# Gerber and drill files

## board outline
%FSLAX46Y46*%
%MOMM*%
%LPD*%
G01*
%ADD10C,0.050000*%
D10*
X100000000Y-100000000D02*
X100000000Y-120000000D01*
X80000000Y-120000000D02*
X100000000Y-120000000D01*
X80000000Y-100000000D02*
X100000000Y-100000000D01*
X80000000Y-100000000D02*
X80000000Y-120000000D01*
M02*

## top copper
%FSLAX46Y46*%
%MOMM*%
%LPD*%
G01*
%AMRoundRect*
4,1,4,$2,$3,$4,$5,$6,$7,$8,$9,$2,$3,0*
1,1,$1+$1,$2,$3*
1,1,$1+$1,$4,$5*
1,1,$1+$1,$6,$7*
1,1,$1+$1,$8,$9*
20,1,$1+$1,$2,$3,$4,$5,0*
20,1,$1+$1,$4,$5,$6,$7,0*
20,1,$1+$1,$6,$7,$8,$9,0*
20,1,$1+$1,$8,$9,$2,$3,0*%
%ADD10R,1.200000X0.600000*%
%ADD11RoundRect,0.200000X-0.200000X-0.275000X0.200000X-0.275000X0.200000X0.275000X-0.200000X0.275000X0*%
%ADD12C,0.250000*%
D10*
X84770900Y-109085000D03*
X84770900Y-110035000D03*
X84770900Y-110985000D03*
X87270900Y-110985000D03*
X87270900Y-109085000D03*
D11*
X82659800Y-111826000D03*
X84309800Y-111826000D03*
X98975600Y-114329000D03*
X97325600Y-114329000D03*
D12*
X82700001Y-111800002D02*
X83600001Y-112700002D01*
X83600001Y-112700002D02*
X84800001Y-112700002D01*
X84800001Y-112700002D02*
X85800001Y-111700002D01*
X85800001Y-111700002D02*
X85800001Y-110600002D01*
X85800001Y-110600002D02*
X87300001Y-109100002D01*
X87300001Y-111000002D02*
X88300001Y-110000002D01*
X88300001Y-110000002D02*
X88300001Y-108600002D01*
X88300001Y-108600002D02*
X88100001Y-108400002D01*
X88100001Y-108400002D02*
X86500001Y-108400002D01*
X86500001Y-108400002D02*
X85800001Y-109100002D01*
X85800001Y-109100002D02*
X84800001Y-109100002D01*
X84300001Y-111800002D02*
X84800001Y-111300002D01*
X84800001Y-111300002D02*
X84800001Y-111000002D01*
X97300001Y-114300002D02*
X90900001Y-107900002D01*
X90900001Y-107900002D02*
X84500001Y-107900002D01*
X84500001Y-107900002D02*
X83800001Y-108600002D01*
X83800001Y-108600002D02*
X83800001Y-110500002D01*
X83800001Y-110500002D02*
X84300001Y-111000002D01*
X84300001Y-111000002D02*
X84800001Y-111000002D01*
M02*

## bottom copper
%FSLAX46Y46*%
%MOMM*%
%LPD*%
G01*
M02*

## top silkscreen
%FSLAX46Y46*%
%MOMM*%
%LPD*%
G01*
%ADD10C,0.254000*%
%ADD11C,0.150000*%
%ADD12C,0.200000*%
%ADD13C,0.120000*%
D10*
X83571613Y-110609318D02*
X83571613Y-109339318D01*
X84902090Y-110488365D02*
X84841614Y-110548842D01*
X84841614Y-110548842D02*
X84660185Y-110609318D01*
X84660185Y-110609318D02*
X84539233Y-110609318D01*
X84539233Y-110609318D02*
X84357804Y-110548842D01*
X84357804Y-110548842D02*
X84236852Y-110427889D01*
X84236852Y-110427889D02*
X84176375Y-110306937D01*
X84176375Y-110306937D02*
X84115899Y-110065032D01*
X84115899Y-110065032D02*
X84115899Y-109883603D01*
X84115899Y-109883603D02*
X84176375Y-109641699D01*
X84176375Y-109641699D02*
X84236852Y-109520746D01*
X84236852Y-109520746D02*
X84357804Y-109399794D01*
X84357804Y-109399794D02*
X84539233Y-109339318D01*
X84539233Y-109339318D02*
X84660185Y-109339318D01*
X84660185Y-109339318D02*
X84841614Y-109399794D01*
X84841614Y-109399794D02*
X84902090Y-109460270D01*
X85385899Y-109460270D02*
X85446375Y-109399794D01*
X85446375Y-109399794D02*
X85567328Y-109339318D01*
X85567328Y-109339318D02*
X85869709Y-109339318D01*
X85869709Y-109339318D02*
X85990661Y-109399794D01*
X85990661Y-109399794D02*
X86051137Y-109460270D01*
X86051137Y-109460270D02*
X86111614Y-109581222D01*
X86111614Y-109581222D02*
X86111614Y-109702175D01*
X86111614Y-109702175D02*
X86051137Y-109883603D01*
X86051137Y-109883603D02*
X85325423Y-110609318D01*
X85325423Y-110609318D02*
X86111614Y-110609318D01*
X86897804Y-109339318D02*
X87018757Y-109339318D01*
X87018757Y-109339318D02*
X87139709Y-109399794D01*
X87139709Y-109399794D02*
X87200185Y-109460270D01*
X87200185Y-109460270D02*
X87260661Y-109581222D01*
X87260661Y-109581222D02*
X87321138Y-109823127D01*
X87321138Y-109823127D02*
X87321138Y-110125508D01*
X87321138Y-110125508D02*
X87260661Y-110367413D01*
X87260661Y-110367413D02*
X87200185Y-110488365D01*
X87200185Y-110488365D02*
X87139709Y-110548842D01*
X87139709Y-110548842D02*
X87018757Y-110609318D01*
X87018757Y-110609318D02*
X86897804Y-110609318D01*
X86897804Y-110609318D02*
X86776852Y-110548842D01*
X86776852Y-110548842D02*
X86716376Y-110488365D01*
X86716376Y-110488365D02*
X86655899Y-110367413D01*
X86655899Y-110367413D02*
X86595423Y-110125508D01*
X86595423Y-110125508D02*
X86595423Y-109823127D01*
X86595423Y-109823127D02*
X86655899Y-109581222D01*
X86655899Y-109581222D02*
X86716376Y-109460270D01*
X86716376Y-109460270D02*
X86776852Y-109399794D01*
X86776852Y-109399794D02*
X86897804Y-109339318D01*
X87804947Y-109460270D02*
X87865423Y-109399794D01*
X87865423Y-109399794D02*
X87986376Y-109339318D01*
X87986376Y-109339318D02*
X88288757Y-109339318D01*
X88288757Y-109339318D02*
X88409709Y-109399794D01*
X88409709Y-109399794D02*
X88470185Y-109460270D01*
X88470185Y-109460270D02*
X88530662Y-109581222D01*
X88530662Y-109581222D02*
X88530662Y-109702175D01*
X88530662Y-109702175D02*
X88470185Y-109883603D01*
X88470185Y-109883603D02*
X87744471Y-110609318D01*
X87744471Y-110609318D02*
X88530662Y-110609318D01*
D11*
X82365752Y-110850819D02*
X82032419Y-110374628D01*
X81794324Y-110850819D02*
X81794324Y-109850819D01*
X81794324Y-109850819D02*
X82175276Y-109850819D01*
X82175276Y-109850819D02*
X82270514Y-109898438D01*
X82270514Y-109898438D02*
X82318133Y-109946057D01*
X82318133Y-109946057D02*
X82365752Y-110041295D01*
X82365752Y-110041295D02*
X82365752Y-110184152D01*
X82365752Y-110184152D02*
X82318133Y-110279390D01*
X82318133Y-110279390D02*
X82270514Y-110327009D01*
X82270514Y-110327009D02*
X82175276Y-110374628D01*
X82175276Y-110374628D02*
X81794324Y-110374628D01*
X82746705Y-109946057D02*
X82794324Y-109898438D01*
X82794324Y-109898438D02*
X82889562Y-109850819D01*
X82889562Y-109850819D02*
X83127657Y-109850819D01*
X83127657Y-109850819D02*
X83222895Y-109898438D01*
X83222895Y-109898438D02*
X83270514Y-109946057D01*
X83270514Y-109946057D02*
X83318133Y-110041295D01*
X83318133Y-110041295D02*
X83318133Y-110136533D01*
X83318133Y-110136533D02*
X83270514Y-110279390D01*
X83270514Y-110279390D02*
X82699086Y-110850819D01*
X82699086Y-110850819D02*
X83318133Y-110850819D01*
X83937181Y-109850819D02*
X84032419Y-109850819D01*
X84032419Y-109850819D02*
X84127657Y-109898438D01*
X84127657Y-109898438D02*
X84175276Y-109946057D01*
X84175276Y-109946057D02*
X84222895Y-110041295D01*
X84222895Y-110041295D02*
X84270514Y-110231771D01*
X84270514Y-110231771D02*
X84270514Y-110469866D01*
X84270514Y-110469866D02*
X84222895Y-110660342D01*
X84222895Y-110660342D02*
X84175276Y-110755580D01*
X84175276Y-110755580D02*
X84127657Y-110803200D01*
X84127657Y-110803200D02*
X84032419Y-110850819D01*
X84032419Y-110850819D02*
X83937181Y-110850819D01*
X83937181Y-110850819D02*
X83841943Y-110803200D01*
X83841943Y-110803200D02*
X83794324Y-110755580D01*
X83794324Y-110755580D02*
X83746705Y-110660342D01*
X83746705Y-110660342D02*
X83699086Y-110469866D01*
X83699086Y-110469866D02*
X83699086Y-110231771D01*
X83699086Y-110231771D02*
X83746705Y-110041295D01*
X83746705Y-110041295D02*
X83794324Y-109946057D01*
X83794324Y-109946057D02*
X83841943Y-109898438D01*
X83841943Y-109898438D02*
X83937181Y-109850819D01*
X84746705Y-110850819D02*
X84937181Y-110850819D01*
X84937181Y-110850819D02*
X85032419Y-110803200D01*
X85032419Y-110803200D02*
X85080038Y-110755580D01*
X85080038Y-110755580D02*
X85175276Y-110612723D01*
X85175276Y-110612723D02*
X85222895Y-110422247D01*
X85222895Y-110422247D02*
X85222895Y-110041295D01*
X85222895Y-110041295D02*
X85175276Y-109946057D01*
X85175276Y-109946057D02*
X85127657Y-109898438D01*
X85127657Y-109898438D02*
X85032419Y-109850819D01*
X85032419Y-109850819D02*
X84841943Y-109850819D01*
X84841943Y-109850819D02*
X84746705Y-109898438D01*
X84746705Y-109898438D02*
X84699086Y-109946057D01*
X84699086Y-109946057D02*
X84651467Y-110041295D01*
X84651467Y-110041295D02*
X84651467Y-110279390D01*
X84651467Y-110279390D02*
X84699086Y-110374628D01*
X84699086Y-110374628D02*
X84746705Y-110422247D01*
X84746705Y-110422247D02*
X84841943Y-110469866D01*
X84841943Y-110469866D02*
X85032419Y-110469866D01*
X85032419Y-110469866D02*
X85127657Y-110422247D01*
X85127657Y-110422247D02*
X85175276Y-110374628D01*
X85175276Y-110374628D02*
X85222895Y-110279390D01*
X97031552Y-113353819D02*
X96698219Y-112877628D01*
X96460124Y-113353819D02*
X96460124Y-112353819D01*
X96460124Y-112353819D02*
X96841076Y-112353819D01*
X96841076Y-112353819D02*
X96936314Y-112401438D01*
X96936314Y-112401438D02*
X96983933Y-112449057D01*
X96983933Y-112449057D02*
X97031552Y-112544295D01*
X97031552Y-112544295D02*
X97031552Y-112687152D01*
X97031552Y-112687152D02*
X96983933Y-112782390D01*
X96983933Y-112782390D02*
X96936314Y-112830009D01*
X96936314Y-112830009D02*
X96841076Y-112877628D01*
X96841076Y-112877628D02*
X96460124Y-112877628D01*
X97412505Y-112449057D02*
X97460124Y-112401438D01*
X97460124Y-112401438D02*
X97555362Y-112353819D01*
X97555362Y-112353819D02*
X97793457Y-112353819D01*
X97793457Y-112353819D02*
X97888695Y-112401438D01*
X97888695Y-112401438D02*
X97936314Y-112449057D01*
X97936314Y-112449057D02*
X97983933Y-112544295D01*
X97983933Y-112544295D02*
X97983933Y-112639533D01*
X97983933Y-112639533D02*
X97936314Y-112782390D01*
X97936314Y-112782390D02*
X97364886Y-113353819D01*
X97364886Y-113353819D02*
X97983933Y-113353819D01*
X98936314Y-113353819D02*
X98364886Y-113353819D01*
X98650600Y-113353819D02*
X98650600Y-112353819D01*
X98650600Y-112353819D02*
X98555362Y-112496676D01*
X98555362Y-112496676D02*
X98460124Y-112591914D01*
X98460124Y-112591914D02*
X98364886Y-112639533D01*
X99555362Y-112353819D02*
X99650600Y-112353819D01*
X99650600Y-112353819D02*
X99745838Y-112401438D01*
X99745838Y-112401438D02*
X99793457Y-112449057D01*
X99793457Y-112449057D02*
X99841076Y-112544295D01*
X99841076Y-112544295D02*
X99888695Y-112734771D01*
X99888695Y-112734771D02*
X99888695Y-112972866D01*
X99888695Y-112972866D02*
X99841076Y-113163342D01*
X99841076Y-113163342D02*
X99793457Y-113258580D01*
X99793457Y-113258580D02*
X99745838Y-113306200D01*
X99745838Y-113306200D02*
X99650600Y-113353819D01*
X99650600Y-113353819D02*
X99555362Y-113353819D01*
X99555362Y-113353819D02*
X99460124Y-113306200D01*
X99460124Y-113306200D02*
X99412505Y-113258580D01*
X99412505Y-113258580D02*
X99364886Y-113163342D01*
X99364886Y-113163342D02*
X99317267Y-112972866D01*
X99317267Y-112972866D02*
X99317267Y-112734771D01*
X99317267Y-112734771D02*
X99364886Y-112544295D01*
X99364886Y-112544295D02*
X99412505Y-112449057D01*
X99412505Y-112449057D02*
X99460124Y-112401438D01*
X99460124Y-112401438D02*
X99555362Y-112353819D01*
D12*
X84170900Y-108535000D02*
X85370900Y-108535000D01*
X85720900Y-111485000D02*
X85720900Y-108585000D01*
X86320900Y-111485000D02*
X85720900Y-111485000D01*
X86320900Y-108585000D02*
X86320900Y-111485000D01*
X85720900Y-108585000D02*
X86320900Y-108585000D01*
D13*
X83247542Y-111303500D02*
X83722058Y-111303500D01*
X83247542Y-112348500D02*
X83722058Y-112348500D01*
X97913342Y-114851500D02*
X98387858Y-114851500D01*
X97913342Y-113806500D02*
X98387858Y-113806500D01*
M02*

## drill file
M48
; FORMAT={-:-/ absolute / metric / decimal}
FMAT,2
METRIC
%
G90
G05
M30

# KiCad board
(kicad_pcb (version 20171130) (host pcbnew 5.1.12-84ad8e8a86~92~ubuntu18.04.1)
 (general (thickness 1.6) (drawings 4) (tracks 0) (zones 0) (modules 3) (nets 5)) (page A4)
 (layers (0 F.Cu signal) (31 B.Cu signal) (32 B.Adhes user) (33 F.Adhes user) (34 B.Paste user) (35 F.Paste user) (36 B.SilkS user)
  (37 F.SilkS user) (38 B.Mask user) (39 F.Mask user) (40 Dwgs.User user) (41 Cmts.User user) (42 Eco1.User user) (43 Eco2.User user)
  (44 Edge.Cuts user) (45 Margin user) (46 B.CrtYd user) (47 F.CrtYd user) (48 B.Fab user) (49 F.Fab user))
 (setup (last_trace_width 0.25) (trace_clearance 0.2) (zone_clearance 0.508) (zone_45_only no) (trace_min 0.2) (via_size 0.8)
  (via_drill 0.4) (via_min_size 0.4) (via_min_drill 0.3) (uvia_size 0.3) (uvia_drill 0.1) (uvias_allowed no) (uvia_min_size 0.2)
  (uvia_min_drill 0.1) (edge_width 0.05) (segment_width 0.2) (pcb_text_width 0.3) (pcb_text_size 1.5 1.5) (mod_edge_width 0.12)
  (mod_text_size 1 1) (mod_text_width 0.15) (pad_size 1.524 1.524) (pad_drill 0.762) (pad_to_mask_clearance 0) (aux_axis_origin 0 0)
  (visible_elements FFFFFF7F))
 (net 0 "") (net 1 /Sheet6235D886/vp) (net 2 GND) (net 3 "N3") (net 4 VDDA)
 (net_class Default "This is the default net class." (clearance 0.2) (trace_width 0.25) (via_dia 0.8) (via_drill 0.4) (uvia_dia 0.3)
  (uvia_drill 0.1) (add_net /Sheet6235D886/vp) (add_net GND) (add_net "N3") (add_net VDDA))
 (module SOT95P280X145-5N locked (layer F.Cu) (at 86.020900 110.035000)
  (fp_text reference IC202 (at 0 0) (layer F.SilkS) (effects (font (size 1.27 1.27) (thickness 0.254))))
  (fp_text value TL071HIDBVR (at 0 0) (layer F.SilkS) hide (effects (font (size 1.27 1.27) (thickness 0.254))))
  (fp_line (start -1.85 -1.5) (end -0.65 -1.5) (layer F.SilkS) (width 0.2))
  (fp_line (start -0.3 1.45) (end -0.3 -1.45) (layer F.SilkS) (width 0.2))
  (fp_line (start 0.3 1.45) (end -0.3 1.45) (layer F.SilkS) (width 0.2))
  (fp_line (start 0.3 -1.45) (end 0.3 1.45) (layer F.SilkS) (width 0.2))
  (fp_line (start -0.3 -1.45) (end 0.3 -1.45) (layer F.SilkS) (width 0.2))
  (pad 1 smd rect (at -1.25 -0.95 90.000000) (size 0.6 1.2) (layers F.Cu F.Mask F.Paste) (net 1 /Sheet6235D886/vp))
  (pad 2 smd rect (at -1.25 0 90.000000) (size 0.6 1.2) (layers F.Cu F.Mask F.Paste) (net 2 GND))
  (pad 3 smd rect (at -1.25 0.95 90.000000) (size 0.6 1.2) (layers F.Cu F.Mask F.Paste) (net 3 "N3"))
  (pad 4 smd rect (at 1.25 0.95 90.000000) (size 0.6 1.2) (layers F.Cu F.Mask F.Paste) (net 1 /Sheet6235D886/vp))
  (pad 5 smd rect (at 1.25 -0.95 90.000000) (size 0.6 1.2) (layers F.Cu F.Mask F.Paste) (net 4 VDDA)))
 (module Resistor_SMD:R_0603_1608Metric (layer F.Cu) (at 83.484800 111.826000)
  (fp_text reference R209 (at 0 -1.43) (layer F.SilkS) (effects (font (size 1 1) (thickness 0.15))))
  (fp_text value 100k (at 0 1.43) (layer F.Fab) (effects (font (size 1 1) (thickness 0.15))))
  (fp_line (start -0.237258 -0.5225) (end 0.237258 -0.5225) (layer F.SilkS) (width 0.12))
  (fp_line (start -0.237258 0.5225) (end 0.237258 0.5225) (layer F.SilkS) (width 0.12))
  (pad 1 smd roundrect (at -0.825 0) (size 0.8 0.95) (layers F.Cu F.Mask F.Paste) (roundrect_rratio 0.25) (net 4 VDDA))
  (pad 2 smd roundrect (at 0.825 0) (size 0.8 0.95) (layers F.Cu F.Mask F.Paste) (roundrect_rratio 0.25) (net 3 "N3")))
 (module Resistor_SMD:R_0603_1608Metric (layer F.Cu) (at 98.150600 114.329000)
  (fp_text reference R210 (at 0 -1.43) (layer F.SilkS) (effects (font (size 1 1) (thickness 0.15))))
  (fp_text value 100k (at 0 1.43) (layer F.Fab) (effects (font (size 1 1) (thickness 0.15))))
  (fp_line (start -0.237258 0.5225) (end 0.237258 0.5225) (layer F.SilkS) (width 0.12))
  (fp_line (start -0.237258 -0.5225) (end 0.237258 -0.5225) (layer F.SilkS) (width 0.12))
  (pad 2 smd roundrect (at 0.825 0) (size 0.8 0.95) (layers F.Cu F.Mask F.Paste) (roundrect_rratio 0.25) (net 2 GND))
  (pad 1 smd roundrect (at -0.825 0) (size 0.8 0.95) (layers F.Cu F.Mask F.Paste) (roundrect_rratio 0.25) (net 3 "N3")))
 (gr_line (start 100 100) (end 100 120) (layer Edge.Cuts) (width 0.05))
 (gr_line (start 80 120) (end 100 120) (layer Edge.Cuts) (width 0.05))
 (gr_line (start 80 100) (end 100 100) (layer Edge.Cuts) (width 0.05))
 (gr_line (start 80 100) (end 80 120) (layer Edge.Cuts) (width 0.05))
 (segment (start 82.700001 111.800002) (end 83.600001 112.700002) (width 0.250000) (layer F.Cu) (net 4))
 (segment (start 83.600001 112.700002) (end 84.800001 112.700002) (width 0.250000) (layer F.Cu) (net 4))
 (segment (start 84.800001 112.700002) (end 85.800001 111.700002) (width 0.250000) (layer F.Cu) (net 4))
 (segment (start 85.800001 111.700002) (end 85.800001 110.600002) (width 0.250000) (layer F.Cu) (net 4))
 (segment (start 85.800001 110.600002) (end 87.300001 109.100002) (width 0.250000) (layer F.Cu) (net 4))
 (segment (start 87.300001 111.000002) (end 88.300001 110.000002) (width 0.250000) (layer F.Cu) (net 1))
 (segment (start 88.300001 110.000002) (end 88.300001 108.600002) (width 0.250000) (layer F.Cu) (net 1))
 (segment (start 88.300001 108.600002) (end 88.100001 108.400002) (width 0.250000) (layer F.Cu) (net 1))
 (segment (start 88.100001 108.400002) (end 86.500001 108.400002) (width 0.250000) (layer F.Cu) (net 1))
 (segment (start 86.500001 108.400002) (end 85.800001 109.100002) (width 0.250000) (layer F.Cu) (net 1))
 (segment (start 85.800001 109.100002) (end 84.800001 109.100002) (width 0.250000) (layer F.Cu) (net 1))
 (segment (start 84.300001 111.800002) (end 84.800001 111.300002) (width 0.250000) (layer F.Cu) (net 3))
 (segment (start 84.800001 111.300002) (end 84.800001 111.000002) (width 0.250000) (layer F.Cu) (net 3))
 (segment (start 97.300001 114.300002) (end 90.900001 107.900002) (width 0.250000) (layer F.Cu) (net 3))
 (segment (start 90.900001 107.900002) (end 84.500001 107.900002) (width 0.250000) (layer F.Cu) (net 3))
 (segment (start 84.500001 107.900002) (end 83.800001 108.600002) (width 0.250000) (layer F.Cu) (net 3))
 (segment (start 83.800001 108.600002) (end 83.800001 110.500002) (width 0.250000) (layer F.Cu) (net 3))
 (segment (start 83.800001 110.500002) (end 84.300001 111.000002) (width 0.250000) (layer F.Cu) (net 3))
 (segment (start 84.300001 111.000002) (end 84.800001 111.000002) (width 0.250000) (layer F.Cu) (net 3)))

